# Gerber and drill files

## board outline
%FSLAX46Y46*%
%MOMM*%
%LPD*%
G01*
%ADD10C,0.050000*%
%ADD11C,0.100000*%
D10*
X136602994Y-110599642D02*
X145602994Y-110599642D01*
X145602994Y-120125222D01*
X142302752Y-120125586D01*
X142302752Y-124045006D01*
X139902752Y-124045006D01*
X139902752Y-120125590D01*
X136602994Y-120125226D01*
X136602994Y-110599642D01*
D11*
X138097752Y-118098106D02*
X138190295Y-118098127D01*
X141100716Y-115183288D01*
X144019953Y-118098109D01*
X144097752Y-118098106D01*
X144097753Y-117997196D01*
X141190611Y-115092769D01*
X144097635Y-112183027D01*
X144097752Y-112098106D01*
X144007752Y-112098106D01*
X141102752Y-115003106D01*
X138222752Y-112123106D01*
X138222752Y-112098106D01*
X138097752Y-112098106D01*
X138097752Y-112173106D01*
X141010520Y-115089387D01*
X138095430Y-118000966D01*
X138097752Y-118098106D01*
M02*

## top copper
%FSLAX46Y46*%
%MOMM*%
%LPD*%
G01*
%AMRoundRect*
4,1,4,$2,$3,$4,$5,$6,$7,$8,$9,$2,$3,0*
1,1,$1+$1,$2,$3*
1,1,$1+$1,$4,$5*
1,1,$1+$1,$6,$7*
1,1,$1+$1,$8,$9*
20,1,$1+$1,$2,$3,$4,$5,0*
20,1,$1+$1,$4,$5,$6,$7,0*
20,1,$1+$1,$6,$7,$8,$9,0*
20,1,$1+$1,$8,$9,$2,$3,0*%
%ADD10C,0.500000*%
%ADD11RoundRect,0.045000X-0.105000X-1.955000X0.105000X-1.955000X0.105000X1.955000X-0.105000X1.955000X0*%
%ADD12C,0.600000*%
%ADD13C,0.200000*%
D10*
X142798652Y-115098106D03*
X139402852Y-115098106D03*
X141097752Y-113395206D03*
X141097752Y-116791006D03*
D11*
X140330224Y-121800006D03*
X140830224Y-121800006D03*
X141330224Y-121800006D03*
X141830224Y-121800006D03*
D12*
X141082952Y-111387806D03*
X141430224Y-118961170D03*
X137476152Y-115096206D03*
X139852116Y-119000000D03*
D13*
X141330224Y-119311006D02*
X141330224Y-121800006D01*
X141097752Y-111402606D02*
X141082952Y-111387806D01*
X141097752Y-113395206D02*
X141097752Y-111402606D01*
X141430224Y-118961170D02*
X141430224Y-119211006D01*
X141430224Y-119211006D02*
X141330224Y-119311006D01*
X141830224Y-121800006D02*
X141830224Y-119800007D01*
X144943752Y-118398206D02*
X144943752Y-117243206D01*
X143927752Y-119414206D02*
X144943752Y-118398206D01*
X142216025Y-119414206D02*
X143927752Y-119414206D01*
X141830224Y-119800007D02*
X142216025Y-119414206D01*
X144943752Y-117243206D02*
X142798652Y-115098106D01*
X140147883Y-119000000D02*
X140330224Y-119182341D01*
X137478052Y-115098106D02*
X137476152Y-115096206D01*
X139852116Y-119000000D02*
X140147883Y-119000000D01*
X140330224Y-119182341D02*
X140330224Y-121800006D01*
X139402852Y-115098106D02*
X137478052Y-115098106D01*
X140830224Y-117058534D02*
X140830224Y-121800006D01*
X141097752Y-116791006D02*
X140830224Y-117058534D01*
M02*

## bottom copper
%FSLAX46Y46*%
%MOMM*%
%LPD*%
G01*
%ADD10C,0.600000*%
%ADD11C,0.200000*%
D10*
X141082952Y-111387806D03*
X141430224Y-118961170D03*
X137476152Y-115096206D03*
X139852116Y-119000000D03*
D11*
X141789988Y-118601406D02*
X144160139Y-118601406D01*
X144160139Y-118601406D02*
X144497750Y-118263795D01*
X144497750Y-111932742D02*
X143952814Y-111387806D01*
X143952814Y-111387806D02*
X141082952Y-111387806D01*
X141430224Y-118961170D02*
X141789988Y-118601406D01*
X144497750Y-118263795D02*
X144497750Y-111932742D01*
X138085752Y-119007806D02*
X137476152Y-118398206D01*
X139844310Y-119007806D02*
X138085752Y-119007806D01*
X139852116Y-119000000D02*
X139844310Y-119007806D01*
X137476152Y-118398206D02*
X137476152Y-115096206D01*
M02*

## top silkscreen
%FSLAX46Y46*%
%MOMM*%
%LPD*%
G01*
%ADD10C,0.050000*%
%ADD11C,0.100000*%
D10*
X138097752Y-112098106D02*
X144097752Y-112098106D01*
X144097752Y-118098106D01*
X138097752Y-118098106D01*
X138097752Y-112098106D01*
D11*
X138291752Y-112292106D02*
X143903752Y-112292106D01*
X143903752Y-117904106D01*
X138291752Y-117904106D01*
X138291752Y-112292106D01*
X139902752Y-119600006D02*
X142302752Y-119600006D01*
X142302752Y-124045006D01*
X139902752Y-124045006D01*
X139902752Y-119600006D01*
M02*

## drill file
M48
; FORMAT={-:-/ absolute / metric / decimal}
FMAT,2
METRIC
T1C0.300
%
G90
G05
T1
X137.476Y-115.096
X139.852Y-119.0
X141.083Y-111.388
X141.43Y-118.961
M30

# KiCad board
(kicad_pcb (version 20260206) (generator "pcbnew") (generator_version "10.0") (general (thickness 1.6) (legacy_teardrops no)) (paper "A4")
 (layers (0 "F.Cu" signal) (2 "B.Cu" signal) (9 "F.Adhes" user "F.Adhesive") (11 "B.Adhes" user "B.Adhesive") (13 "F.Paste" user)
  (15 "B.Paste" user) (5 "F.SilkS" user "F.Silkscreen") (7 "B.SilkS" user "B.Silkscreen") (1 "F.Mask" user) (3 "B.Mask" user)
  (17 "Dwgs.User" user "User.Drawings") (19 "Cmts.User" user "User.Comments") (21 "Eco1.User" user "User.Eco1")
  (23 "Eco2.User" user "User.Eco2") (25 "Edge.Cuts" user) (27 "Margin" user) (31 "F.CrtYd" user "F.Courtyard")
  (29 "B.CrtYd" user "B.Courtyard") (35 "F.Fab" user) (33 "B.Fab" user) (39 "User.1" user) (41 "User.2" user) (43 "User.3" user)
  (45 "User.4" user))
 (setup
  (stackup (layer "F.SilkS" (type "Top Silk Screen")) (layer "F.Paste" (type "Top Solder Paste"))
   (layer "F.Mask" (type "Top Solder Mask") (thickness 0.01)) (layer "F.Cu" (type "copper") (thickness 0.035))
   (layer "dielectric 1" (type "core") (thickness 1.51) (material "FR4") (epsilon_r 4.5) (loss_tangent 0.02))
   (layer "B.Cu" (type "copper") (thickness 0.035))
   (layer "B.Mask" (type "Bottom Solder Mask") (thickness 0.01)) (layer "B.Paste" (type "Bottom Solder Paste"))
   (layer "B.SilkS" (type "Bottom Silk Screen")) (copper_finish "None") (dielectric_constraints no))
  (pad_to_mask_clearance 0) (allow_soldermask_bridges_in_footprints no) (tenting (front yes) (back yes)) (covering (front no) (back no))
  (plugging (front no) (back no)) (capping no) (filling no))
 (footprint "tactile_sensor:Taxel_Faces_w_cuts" (layer "F.Cu") (at 141.097752 115.098106)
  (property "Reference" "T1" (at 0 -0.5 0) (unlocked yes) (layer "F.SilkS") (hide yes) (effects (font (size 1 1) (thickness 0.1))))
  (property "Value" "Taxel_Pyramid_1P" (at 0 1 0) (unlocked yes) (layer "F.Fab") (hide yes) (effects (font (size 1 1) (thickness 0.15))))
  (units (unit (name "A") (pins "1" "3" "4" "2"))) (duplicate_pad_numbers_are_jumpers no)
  (fp_rect (start -3 -3) (end 3 3) (stroke (width 0.05) (type solid)) (fill no) (layer "F.SilkS"))
  (fp_rect (start -2.806 -2.806) (end 2.806 2.806) (stroke (width 0.1) (type solid)) (fill no) (layer "F.SilkS"))
  (fp_poly
   (pts (xy -3 3) (xy -2.907457 3.000021) (xy 0.002964 0.085182) (xy 2.922201 3.000003) (xy 3 3) (xy 3.000001 2.89909)
    (xy 0.092859 -0.005337) (xy 2.999883 -2.915079) (xy 3 -3) (xy 2.91 -3) (xy 0.005 -0.095) (xy -2.875 -2.975) (xy -2.875 -3) (xy -3 -3)
    (xy -3 -2.925) (xy -0.087232 -0.008719) (xy -3.002322 2.90286))
   (stroke (width 0.1) (type solid)) (fill no) (layer "Edge.Cuts"))
  (pad "1" smd circle (at 1.7009 0 90) (size 0.5 0.5) (layers "F.Cu" "F.Mask") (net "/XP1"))
  (pad "2" smd circle (at -1.6949 0 270) (size 0.5 0.5) (layers "F.Cu" "F.Mask") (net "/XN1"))
  (pad "3" smd circle (at 0 -1.7029) (size 0.5 0.5) (layers "F.Cu" "F.Mask") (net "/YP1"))
  (pad "4" smd circle (at 0 1.6929) (size 0.5 0.5) (layers "F.Cu" "F.Mask") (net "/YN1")))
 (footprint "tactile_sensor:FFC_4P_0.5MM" (layer "F.Cu") (at 141.100224 123.810006)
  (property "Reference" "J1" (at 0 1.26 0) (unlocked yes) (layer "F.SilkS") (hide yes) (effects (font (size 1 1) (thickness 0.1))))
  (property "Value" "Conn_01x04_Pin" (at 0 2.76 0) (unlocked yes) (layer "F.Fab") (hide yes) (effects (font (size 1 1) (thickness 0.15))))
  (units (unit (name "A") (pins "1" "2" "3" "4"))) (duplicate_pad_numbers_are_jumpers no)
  (fp_rect (start -1.197472 -4.21) (end 1.202528 0.235) (stroke (width 0.1) (type default)) (fill no) (layer "F.SilkS"))
  (pad "1" smd roundrect (at -0.77 -2.01) (size 0.3 4) (layers "F.Cu" "F.Mask" "F.Paste") (roundrect_rratio 0.15) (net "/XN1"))
  (pad "2" smd roundrect (at -0.27 -2.01) (size 0.3 4) (layers "F.Cu" "F.Mask" "F.Paste") (roundrect_rratio 0.15) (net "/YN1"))
  (pad "3" smd roundrect (at 0.23 -2.01) (size 0.3 4) (layers "F.Cu" "F.Mask" "F.Paste") (roundrect_rratio 0.15) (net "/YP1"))
  (pad "4" smd roundrect (at 0.73 -2.01) (size 0.3 4) (layers "F.Cu" "F.Mask" "F.Paste") (roundrect_rratio 0.15) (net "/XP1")))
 (gr_poly
  (pts (xy 136.602994 110.599642) (xy 145.602994 110.599642) (xy 145.602994 120.125222) (xy 142.302752 120.125586)
   (xy 142.302752 124.045006) (xy 139.902752 124.045006) (xy 139.902752 120.12559) (xy 136.602994 120.125226))
  (stroke (width 0.05) (type solid)) (fill no) (layer "Edge.Cuts"))
 (segment (start 141.330224 119.311006) (end 141.330224 121.800006) (width 0.2) (layer "F.Cu") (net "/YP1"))
 (segment (start 141.097752 111.402606) (end 141.082952 111.387806) (width 0.2) (layer "F.Cu") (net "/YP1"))
 (segment (start 141.097752 113.395206) (end 141.097752 111.402606) (width 0.2) (layer "F.Cu") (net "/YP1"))
 (segment (start 141.430224 118.96117) (end 141.430224 119.211006) (width 0.2) (layer "F.Cu") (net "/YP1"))
 (segment (start 141.430224 119.211006) (end 141.330224 119.311006) (width 0.2) (layer "F.Cu") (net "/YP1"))
 (via (at 141.082952 111.387806) (size 0.6) (drill 0.3) (layers "F.Cu" "B.Cu") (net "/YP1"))
 (via (at 141.430224 118.96117) (size 0.6) (drill 0.3) (layers "F.Cu" "B.Cu") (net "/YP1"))
 (segment (start 141.789988 118.601406) (end 144.160139 118.601406) (width 0.2) (layer "B.Cu") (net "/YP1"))
 (segment (start 144.160139 118.601406) (end 144.49775 118.263795) (width 0.2) (layer "B.Cu") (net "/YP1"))
 (segment (start 144.49775 111.932742) (end 143.952814 111.387806) (width 0.2) (layer "B.Cu") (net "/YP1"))
 (segment (start 143.952814 111.387806) (end 141.082952 111.387806) (width 0.2) (layer "B.Cu") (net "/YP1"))
 (segment (start 141.430224 118.96117) (end 141.789988 118.601406) (width 0.2) (layer "B.Cu") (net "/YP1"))
 (segment (start 144.49775 118.263795) (end 144.49775 111.932742) (width 0.2) (layer "B.Cu") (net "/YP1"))
 (segment (start 141.830224 121.800006) (end 141.830224 119.800007) (width 0.2) (layer "F.Cu") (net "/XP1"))
 (segment (start 144.943752 118.398206) (end 144.943752 117.243206) (width 0.2) (layer "F.Cu") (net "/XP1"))
 (segment (start 143.927752 119.414206) (end 144.943752 118.398206) (width 0.2) (layer "F.Cu") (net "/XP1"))
 (segment (start 142.216025 119.414206) (end 143.927752 119.414206) (width 0.2) (layer "F.Cu") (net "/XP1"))
 (segment (start 141.830224 119.800007) (end 142.216025 119.414206) (width 0.2) (layer "F.Cu") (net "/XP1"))
 (segment (start 144.943752 117.243206) (end 142.798652 115.098106) (width 0.2) (layer "F.Cu") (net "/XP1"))
 (segment (start 140.147883 119) (end 140.330224 119.182341) (width 0.2) (layer "F.Cu") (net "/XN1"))
 (segment (start 137.478052 115.098106) (end 137.476152 115.096206) (width 0.2) (layer "F.Cu") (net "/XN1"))
 (segment (start 139.852116 119) (end 140.147883 119) (width 0.2) (layer "F.Cu") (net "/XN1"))
 (segment (start 140.330224 119.182341) (end 140.330224 121.800006) (width 0.2) (layer "F.Cu") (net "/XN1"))
 (segment (start 139.402852 115.098106) (end 137.478052 115.098106) (width 0.2) (layer "F.Cu") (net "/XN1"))
 (via (at 137.476152 115.096206) (size 0.6) (drill 0.3) (layers "F.Cu" "B.Cu") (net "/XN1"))
 (via (at 139.852116 119) (size 0.6) (drill 0.3) (layers "F.Cu" "B.Cu") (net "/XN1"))
 (segment (start 138.085752 119.007806) (end 137.476152 118.398206) (width 0.2) (layer "B.Cu") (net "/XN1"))
 (segment (start 139.84431 119.007806) (end 138.085752 119.007806) (width 0.2) (layer "B.Cu") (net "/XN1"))
 (segment (start 139.852116 119) (end 139.84431 119.007806) (width 0.2) (layer "B.Cu") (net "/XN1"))
 (segment (start 137.476152 118.398206) (end 137.476152 115.096206) (width 0.2) (layer "B.Cu") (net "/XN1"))
 (segment (start 140.830224 117.058534) (end 140.830224 121.800006) (width 0.2) (layer "F.Cu") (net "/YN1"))
 (segment (start 141.097752 116.791006) (end 140.830224 117.058534) (width 0.2) (layer "F.Cu") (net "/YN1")))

